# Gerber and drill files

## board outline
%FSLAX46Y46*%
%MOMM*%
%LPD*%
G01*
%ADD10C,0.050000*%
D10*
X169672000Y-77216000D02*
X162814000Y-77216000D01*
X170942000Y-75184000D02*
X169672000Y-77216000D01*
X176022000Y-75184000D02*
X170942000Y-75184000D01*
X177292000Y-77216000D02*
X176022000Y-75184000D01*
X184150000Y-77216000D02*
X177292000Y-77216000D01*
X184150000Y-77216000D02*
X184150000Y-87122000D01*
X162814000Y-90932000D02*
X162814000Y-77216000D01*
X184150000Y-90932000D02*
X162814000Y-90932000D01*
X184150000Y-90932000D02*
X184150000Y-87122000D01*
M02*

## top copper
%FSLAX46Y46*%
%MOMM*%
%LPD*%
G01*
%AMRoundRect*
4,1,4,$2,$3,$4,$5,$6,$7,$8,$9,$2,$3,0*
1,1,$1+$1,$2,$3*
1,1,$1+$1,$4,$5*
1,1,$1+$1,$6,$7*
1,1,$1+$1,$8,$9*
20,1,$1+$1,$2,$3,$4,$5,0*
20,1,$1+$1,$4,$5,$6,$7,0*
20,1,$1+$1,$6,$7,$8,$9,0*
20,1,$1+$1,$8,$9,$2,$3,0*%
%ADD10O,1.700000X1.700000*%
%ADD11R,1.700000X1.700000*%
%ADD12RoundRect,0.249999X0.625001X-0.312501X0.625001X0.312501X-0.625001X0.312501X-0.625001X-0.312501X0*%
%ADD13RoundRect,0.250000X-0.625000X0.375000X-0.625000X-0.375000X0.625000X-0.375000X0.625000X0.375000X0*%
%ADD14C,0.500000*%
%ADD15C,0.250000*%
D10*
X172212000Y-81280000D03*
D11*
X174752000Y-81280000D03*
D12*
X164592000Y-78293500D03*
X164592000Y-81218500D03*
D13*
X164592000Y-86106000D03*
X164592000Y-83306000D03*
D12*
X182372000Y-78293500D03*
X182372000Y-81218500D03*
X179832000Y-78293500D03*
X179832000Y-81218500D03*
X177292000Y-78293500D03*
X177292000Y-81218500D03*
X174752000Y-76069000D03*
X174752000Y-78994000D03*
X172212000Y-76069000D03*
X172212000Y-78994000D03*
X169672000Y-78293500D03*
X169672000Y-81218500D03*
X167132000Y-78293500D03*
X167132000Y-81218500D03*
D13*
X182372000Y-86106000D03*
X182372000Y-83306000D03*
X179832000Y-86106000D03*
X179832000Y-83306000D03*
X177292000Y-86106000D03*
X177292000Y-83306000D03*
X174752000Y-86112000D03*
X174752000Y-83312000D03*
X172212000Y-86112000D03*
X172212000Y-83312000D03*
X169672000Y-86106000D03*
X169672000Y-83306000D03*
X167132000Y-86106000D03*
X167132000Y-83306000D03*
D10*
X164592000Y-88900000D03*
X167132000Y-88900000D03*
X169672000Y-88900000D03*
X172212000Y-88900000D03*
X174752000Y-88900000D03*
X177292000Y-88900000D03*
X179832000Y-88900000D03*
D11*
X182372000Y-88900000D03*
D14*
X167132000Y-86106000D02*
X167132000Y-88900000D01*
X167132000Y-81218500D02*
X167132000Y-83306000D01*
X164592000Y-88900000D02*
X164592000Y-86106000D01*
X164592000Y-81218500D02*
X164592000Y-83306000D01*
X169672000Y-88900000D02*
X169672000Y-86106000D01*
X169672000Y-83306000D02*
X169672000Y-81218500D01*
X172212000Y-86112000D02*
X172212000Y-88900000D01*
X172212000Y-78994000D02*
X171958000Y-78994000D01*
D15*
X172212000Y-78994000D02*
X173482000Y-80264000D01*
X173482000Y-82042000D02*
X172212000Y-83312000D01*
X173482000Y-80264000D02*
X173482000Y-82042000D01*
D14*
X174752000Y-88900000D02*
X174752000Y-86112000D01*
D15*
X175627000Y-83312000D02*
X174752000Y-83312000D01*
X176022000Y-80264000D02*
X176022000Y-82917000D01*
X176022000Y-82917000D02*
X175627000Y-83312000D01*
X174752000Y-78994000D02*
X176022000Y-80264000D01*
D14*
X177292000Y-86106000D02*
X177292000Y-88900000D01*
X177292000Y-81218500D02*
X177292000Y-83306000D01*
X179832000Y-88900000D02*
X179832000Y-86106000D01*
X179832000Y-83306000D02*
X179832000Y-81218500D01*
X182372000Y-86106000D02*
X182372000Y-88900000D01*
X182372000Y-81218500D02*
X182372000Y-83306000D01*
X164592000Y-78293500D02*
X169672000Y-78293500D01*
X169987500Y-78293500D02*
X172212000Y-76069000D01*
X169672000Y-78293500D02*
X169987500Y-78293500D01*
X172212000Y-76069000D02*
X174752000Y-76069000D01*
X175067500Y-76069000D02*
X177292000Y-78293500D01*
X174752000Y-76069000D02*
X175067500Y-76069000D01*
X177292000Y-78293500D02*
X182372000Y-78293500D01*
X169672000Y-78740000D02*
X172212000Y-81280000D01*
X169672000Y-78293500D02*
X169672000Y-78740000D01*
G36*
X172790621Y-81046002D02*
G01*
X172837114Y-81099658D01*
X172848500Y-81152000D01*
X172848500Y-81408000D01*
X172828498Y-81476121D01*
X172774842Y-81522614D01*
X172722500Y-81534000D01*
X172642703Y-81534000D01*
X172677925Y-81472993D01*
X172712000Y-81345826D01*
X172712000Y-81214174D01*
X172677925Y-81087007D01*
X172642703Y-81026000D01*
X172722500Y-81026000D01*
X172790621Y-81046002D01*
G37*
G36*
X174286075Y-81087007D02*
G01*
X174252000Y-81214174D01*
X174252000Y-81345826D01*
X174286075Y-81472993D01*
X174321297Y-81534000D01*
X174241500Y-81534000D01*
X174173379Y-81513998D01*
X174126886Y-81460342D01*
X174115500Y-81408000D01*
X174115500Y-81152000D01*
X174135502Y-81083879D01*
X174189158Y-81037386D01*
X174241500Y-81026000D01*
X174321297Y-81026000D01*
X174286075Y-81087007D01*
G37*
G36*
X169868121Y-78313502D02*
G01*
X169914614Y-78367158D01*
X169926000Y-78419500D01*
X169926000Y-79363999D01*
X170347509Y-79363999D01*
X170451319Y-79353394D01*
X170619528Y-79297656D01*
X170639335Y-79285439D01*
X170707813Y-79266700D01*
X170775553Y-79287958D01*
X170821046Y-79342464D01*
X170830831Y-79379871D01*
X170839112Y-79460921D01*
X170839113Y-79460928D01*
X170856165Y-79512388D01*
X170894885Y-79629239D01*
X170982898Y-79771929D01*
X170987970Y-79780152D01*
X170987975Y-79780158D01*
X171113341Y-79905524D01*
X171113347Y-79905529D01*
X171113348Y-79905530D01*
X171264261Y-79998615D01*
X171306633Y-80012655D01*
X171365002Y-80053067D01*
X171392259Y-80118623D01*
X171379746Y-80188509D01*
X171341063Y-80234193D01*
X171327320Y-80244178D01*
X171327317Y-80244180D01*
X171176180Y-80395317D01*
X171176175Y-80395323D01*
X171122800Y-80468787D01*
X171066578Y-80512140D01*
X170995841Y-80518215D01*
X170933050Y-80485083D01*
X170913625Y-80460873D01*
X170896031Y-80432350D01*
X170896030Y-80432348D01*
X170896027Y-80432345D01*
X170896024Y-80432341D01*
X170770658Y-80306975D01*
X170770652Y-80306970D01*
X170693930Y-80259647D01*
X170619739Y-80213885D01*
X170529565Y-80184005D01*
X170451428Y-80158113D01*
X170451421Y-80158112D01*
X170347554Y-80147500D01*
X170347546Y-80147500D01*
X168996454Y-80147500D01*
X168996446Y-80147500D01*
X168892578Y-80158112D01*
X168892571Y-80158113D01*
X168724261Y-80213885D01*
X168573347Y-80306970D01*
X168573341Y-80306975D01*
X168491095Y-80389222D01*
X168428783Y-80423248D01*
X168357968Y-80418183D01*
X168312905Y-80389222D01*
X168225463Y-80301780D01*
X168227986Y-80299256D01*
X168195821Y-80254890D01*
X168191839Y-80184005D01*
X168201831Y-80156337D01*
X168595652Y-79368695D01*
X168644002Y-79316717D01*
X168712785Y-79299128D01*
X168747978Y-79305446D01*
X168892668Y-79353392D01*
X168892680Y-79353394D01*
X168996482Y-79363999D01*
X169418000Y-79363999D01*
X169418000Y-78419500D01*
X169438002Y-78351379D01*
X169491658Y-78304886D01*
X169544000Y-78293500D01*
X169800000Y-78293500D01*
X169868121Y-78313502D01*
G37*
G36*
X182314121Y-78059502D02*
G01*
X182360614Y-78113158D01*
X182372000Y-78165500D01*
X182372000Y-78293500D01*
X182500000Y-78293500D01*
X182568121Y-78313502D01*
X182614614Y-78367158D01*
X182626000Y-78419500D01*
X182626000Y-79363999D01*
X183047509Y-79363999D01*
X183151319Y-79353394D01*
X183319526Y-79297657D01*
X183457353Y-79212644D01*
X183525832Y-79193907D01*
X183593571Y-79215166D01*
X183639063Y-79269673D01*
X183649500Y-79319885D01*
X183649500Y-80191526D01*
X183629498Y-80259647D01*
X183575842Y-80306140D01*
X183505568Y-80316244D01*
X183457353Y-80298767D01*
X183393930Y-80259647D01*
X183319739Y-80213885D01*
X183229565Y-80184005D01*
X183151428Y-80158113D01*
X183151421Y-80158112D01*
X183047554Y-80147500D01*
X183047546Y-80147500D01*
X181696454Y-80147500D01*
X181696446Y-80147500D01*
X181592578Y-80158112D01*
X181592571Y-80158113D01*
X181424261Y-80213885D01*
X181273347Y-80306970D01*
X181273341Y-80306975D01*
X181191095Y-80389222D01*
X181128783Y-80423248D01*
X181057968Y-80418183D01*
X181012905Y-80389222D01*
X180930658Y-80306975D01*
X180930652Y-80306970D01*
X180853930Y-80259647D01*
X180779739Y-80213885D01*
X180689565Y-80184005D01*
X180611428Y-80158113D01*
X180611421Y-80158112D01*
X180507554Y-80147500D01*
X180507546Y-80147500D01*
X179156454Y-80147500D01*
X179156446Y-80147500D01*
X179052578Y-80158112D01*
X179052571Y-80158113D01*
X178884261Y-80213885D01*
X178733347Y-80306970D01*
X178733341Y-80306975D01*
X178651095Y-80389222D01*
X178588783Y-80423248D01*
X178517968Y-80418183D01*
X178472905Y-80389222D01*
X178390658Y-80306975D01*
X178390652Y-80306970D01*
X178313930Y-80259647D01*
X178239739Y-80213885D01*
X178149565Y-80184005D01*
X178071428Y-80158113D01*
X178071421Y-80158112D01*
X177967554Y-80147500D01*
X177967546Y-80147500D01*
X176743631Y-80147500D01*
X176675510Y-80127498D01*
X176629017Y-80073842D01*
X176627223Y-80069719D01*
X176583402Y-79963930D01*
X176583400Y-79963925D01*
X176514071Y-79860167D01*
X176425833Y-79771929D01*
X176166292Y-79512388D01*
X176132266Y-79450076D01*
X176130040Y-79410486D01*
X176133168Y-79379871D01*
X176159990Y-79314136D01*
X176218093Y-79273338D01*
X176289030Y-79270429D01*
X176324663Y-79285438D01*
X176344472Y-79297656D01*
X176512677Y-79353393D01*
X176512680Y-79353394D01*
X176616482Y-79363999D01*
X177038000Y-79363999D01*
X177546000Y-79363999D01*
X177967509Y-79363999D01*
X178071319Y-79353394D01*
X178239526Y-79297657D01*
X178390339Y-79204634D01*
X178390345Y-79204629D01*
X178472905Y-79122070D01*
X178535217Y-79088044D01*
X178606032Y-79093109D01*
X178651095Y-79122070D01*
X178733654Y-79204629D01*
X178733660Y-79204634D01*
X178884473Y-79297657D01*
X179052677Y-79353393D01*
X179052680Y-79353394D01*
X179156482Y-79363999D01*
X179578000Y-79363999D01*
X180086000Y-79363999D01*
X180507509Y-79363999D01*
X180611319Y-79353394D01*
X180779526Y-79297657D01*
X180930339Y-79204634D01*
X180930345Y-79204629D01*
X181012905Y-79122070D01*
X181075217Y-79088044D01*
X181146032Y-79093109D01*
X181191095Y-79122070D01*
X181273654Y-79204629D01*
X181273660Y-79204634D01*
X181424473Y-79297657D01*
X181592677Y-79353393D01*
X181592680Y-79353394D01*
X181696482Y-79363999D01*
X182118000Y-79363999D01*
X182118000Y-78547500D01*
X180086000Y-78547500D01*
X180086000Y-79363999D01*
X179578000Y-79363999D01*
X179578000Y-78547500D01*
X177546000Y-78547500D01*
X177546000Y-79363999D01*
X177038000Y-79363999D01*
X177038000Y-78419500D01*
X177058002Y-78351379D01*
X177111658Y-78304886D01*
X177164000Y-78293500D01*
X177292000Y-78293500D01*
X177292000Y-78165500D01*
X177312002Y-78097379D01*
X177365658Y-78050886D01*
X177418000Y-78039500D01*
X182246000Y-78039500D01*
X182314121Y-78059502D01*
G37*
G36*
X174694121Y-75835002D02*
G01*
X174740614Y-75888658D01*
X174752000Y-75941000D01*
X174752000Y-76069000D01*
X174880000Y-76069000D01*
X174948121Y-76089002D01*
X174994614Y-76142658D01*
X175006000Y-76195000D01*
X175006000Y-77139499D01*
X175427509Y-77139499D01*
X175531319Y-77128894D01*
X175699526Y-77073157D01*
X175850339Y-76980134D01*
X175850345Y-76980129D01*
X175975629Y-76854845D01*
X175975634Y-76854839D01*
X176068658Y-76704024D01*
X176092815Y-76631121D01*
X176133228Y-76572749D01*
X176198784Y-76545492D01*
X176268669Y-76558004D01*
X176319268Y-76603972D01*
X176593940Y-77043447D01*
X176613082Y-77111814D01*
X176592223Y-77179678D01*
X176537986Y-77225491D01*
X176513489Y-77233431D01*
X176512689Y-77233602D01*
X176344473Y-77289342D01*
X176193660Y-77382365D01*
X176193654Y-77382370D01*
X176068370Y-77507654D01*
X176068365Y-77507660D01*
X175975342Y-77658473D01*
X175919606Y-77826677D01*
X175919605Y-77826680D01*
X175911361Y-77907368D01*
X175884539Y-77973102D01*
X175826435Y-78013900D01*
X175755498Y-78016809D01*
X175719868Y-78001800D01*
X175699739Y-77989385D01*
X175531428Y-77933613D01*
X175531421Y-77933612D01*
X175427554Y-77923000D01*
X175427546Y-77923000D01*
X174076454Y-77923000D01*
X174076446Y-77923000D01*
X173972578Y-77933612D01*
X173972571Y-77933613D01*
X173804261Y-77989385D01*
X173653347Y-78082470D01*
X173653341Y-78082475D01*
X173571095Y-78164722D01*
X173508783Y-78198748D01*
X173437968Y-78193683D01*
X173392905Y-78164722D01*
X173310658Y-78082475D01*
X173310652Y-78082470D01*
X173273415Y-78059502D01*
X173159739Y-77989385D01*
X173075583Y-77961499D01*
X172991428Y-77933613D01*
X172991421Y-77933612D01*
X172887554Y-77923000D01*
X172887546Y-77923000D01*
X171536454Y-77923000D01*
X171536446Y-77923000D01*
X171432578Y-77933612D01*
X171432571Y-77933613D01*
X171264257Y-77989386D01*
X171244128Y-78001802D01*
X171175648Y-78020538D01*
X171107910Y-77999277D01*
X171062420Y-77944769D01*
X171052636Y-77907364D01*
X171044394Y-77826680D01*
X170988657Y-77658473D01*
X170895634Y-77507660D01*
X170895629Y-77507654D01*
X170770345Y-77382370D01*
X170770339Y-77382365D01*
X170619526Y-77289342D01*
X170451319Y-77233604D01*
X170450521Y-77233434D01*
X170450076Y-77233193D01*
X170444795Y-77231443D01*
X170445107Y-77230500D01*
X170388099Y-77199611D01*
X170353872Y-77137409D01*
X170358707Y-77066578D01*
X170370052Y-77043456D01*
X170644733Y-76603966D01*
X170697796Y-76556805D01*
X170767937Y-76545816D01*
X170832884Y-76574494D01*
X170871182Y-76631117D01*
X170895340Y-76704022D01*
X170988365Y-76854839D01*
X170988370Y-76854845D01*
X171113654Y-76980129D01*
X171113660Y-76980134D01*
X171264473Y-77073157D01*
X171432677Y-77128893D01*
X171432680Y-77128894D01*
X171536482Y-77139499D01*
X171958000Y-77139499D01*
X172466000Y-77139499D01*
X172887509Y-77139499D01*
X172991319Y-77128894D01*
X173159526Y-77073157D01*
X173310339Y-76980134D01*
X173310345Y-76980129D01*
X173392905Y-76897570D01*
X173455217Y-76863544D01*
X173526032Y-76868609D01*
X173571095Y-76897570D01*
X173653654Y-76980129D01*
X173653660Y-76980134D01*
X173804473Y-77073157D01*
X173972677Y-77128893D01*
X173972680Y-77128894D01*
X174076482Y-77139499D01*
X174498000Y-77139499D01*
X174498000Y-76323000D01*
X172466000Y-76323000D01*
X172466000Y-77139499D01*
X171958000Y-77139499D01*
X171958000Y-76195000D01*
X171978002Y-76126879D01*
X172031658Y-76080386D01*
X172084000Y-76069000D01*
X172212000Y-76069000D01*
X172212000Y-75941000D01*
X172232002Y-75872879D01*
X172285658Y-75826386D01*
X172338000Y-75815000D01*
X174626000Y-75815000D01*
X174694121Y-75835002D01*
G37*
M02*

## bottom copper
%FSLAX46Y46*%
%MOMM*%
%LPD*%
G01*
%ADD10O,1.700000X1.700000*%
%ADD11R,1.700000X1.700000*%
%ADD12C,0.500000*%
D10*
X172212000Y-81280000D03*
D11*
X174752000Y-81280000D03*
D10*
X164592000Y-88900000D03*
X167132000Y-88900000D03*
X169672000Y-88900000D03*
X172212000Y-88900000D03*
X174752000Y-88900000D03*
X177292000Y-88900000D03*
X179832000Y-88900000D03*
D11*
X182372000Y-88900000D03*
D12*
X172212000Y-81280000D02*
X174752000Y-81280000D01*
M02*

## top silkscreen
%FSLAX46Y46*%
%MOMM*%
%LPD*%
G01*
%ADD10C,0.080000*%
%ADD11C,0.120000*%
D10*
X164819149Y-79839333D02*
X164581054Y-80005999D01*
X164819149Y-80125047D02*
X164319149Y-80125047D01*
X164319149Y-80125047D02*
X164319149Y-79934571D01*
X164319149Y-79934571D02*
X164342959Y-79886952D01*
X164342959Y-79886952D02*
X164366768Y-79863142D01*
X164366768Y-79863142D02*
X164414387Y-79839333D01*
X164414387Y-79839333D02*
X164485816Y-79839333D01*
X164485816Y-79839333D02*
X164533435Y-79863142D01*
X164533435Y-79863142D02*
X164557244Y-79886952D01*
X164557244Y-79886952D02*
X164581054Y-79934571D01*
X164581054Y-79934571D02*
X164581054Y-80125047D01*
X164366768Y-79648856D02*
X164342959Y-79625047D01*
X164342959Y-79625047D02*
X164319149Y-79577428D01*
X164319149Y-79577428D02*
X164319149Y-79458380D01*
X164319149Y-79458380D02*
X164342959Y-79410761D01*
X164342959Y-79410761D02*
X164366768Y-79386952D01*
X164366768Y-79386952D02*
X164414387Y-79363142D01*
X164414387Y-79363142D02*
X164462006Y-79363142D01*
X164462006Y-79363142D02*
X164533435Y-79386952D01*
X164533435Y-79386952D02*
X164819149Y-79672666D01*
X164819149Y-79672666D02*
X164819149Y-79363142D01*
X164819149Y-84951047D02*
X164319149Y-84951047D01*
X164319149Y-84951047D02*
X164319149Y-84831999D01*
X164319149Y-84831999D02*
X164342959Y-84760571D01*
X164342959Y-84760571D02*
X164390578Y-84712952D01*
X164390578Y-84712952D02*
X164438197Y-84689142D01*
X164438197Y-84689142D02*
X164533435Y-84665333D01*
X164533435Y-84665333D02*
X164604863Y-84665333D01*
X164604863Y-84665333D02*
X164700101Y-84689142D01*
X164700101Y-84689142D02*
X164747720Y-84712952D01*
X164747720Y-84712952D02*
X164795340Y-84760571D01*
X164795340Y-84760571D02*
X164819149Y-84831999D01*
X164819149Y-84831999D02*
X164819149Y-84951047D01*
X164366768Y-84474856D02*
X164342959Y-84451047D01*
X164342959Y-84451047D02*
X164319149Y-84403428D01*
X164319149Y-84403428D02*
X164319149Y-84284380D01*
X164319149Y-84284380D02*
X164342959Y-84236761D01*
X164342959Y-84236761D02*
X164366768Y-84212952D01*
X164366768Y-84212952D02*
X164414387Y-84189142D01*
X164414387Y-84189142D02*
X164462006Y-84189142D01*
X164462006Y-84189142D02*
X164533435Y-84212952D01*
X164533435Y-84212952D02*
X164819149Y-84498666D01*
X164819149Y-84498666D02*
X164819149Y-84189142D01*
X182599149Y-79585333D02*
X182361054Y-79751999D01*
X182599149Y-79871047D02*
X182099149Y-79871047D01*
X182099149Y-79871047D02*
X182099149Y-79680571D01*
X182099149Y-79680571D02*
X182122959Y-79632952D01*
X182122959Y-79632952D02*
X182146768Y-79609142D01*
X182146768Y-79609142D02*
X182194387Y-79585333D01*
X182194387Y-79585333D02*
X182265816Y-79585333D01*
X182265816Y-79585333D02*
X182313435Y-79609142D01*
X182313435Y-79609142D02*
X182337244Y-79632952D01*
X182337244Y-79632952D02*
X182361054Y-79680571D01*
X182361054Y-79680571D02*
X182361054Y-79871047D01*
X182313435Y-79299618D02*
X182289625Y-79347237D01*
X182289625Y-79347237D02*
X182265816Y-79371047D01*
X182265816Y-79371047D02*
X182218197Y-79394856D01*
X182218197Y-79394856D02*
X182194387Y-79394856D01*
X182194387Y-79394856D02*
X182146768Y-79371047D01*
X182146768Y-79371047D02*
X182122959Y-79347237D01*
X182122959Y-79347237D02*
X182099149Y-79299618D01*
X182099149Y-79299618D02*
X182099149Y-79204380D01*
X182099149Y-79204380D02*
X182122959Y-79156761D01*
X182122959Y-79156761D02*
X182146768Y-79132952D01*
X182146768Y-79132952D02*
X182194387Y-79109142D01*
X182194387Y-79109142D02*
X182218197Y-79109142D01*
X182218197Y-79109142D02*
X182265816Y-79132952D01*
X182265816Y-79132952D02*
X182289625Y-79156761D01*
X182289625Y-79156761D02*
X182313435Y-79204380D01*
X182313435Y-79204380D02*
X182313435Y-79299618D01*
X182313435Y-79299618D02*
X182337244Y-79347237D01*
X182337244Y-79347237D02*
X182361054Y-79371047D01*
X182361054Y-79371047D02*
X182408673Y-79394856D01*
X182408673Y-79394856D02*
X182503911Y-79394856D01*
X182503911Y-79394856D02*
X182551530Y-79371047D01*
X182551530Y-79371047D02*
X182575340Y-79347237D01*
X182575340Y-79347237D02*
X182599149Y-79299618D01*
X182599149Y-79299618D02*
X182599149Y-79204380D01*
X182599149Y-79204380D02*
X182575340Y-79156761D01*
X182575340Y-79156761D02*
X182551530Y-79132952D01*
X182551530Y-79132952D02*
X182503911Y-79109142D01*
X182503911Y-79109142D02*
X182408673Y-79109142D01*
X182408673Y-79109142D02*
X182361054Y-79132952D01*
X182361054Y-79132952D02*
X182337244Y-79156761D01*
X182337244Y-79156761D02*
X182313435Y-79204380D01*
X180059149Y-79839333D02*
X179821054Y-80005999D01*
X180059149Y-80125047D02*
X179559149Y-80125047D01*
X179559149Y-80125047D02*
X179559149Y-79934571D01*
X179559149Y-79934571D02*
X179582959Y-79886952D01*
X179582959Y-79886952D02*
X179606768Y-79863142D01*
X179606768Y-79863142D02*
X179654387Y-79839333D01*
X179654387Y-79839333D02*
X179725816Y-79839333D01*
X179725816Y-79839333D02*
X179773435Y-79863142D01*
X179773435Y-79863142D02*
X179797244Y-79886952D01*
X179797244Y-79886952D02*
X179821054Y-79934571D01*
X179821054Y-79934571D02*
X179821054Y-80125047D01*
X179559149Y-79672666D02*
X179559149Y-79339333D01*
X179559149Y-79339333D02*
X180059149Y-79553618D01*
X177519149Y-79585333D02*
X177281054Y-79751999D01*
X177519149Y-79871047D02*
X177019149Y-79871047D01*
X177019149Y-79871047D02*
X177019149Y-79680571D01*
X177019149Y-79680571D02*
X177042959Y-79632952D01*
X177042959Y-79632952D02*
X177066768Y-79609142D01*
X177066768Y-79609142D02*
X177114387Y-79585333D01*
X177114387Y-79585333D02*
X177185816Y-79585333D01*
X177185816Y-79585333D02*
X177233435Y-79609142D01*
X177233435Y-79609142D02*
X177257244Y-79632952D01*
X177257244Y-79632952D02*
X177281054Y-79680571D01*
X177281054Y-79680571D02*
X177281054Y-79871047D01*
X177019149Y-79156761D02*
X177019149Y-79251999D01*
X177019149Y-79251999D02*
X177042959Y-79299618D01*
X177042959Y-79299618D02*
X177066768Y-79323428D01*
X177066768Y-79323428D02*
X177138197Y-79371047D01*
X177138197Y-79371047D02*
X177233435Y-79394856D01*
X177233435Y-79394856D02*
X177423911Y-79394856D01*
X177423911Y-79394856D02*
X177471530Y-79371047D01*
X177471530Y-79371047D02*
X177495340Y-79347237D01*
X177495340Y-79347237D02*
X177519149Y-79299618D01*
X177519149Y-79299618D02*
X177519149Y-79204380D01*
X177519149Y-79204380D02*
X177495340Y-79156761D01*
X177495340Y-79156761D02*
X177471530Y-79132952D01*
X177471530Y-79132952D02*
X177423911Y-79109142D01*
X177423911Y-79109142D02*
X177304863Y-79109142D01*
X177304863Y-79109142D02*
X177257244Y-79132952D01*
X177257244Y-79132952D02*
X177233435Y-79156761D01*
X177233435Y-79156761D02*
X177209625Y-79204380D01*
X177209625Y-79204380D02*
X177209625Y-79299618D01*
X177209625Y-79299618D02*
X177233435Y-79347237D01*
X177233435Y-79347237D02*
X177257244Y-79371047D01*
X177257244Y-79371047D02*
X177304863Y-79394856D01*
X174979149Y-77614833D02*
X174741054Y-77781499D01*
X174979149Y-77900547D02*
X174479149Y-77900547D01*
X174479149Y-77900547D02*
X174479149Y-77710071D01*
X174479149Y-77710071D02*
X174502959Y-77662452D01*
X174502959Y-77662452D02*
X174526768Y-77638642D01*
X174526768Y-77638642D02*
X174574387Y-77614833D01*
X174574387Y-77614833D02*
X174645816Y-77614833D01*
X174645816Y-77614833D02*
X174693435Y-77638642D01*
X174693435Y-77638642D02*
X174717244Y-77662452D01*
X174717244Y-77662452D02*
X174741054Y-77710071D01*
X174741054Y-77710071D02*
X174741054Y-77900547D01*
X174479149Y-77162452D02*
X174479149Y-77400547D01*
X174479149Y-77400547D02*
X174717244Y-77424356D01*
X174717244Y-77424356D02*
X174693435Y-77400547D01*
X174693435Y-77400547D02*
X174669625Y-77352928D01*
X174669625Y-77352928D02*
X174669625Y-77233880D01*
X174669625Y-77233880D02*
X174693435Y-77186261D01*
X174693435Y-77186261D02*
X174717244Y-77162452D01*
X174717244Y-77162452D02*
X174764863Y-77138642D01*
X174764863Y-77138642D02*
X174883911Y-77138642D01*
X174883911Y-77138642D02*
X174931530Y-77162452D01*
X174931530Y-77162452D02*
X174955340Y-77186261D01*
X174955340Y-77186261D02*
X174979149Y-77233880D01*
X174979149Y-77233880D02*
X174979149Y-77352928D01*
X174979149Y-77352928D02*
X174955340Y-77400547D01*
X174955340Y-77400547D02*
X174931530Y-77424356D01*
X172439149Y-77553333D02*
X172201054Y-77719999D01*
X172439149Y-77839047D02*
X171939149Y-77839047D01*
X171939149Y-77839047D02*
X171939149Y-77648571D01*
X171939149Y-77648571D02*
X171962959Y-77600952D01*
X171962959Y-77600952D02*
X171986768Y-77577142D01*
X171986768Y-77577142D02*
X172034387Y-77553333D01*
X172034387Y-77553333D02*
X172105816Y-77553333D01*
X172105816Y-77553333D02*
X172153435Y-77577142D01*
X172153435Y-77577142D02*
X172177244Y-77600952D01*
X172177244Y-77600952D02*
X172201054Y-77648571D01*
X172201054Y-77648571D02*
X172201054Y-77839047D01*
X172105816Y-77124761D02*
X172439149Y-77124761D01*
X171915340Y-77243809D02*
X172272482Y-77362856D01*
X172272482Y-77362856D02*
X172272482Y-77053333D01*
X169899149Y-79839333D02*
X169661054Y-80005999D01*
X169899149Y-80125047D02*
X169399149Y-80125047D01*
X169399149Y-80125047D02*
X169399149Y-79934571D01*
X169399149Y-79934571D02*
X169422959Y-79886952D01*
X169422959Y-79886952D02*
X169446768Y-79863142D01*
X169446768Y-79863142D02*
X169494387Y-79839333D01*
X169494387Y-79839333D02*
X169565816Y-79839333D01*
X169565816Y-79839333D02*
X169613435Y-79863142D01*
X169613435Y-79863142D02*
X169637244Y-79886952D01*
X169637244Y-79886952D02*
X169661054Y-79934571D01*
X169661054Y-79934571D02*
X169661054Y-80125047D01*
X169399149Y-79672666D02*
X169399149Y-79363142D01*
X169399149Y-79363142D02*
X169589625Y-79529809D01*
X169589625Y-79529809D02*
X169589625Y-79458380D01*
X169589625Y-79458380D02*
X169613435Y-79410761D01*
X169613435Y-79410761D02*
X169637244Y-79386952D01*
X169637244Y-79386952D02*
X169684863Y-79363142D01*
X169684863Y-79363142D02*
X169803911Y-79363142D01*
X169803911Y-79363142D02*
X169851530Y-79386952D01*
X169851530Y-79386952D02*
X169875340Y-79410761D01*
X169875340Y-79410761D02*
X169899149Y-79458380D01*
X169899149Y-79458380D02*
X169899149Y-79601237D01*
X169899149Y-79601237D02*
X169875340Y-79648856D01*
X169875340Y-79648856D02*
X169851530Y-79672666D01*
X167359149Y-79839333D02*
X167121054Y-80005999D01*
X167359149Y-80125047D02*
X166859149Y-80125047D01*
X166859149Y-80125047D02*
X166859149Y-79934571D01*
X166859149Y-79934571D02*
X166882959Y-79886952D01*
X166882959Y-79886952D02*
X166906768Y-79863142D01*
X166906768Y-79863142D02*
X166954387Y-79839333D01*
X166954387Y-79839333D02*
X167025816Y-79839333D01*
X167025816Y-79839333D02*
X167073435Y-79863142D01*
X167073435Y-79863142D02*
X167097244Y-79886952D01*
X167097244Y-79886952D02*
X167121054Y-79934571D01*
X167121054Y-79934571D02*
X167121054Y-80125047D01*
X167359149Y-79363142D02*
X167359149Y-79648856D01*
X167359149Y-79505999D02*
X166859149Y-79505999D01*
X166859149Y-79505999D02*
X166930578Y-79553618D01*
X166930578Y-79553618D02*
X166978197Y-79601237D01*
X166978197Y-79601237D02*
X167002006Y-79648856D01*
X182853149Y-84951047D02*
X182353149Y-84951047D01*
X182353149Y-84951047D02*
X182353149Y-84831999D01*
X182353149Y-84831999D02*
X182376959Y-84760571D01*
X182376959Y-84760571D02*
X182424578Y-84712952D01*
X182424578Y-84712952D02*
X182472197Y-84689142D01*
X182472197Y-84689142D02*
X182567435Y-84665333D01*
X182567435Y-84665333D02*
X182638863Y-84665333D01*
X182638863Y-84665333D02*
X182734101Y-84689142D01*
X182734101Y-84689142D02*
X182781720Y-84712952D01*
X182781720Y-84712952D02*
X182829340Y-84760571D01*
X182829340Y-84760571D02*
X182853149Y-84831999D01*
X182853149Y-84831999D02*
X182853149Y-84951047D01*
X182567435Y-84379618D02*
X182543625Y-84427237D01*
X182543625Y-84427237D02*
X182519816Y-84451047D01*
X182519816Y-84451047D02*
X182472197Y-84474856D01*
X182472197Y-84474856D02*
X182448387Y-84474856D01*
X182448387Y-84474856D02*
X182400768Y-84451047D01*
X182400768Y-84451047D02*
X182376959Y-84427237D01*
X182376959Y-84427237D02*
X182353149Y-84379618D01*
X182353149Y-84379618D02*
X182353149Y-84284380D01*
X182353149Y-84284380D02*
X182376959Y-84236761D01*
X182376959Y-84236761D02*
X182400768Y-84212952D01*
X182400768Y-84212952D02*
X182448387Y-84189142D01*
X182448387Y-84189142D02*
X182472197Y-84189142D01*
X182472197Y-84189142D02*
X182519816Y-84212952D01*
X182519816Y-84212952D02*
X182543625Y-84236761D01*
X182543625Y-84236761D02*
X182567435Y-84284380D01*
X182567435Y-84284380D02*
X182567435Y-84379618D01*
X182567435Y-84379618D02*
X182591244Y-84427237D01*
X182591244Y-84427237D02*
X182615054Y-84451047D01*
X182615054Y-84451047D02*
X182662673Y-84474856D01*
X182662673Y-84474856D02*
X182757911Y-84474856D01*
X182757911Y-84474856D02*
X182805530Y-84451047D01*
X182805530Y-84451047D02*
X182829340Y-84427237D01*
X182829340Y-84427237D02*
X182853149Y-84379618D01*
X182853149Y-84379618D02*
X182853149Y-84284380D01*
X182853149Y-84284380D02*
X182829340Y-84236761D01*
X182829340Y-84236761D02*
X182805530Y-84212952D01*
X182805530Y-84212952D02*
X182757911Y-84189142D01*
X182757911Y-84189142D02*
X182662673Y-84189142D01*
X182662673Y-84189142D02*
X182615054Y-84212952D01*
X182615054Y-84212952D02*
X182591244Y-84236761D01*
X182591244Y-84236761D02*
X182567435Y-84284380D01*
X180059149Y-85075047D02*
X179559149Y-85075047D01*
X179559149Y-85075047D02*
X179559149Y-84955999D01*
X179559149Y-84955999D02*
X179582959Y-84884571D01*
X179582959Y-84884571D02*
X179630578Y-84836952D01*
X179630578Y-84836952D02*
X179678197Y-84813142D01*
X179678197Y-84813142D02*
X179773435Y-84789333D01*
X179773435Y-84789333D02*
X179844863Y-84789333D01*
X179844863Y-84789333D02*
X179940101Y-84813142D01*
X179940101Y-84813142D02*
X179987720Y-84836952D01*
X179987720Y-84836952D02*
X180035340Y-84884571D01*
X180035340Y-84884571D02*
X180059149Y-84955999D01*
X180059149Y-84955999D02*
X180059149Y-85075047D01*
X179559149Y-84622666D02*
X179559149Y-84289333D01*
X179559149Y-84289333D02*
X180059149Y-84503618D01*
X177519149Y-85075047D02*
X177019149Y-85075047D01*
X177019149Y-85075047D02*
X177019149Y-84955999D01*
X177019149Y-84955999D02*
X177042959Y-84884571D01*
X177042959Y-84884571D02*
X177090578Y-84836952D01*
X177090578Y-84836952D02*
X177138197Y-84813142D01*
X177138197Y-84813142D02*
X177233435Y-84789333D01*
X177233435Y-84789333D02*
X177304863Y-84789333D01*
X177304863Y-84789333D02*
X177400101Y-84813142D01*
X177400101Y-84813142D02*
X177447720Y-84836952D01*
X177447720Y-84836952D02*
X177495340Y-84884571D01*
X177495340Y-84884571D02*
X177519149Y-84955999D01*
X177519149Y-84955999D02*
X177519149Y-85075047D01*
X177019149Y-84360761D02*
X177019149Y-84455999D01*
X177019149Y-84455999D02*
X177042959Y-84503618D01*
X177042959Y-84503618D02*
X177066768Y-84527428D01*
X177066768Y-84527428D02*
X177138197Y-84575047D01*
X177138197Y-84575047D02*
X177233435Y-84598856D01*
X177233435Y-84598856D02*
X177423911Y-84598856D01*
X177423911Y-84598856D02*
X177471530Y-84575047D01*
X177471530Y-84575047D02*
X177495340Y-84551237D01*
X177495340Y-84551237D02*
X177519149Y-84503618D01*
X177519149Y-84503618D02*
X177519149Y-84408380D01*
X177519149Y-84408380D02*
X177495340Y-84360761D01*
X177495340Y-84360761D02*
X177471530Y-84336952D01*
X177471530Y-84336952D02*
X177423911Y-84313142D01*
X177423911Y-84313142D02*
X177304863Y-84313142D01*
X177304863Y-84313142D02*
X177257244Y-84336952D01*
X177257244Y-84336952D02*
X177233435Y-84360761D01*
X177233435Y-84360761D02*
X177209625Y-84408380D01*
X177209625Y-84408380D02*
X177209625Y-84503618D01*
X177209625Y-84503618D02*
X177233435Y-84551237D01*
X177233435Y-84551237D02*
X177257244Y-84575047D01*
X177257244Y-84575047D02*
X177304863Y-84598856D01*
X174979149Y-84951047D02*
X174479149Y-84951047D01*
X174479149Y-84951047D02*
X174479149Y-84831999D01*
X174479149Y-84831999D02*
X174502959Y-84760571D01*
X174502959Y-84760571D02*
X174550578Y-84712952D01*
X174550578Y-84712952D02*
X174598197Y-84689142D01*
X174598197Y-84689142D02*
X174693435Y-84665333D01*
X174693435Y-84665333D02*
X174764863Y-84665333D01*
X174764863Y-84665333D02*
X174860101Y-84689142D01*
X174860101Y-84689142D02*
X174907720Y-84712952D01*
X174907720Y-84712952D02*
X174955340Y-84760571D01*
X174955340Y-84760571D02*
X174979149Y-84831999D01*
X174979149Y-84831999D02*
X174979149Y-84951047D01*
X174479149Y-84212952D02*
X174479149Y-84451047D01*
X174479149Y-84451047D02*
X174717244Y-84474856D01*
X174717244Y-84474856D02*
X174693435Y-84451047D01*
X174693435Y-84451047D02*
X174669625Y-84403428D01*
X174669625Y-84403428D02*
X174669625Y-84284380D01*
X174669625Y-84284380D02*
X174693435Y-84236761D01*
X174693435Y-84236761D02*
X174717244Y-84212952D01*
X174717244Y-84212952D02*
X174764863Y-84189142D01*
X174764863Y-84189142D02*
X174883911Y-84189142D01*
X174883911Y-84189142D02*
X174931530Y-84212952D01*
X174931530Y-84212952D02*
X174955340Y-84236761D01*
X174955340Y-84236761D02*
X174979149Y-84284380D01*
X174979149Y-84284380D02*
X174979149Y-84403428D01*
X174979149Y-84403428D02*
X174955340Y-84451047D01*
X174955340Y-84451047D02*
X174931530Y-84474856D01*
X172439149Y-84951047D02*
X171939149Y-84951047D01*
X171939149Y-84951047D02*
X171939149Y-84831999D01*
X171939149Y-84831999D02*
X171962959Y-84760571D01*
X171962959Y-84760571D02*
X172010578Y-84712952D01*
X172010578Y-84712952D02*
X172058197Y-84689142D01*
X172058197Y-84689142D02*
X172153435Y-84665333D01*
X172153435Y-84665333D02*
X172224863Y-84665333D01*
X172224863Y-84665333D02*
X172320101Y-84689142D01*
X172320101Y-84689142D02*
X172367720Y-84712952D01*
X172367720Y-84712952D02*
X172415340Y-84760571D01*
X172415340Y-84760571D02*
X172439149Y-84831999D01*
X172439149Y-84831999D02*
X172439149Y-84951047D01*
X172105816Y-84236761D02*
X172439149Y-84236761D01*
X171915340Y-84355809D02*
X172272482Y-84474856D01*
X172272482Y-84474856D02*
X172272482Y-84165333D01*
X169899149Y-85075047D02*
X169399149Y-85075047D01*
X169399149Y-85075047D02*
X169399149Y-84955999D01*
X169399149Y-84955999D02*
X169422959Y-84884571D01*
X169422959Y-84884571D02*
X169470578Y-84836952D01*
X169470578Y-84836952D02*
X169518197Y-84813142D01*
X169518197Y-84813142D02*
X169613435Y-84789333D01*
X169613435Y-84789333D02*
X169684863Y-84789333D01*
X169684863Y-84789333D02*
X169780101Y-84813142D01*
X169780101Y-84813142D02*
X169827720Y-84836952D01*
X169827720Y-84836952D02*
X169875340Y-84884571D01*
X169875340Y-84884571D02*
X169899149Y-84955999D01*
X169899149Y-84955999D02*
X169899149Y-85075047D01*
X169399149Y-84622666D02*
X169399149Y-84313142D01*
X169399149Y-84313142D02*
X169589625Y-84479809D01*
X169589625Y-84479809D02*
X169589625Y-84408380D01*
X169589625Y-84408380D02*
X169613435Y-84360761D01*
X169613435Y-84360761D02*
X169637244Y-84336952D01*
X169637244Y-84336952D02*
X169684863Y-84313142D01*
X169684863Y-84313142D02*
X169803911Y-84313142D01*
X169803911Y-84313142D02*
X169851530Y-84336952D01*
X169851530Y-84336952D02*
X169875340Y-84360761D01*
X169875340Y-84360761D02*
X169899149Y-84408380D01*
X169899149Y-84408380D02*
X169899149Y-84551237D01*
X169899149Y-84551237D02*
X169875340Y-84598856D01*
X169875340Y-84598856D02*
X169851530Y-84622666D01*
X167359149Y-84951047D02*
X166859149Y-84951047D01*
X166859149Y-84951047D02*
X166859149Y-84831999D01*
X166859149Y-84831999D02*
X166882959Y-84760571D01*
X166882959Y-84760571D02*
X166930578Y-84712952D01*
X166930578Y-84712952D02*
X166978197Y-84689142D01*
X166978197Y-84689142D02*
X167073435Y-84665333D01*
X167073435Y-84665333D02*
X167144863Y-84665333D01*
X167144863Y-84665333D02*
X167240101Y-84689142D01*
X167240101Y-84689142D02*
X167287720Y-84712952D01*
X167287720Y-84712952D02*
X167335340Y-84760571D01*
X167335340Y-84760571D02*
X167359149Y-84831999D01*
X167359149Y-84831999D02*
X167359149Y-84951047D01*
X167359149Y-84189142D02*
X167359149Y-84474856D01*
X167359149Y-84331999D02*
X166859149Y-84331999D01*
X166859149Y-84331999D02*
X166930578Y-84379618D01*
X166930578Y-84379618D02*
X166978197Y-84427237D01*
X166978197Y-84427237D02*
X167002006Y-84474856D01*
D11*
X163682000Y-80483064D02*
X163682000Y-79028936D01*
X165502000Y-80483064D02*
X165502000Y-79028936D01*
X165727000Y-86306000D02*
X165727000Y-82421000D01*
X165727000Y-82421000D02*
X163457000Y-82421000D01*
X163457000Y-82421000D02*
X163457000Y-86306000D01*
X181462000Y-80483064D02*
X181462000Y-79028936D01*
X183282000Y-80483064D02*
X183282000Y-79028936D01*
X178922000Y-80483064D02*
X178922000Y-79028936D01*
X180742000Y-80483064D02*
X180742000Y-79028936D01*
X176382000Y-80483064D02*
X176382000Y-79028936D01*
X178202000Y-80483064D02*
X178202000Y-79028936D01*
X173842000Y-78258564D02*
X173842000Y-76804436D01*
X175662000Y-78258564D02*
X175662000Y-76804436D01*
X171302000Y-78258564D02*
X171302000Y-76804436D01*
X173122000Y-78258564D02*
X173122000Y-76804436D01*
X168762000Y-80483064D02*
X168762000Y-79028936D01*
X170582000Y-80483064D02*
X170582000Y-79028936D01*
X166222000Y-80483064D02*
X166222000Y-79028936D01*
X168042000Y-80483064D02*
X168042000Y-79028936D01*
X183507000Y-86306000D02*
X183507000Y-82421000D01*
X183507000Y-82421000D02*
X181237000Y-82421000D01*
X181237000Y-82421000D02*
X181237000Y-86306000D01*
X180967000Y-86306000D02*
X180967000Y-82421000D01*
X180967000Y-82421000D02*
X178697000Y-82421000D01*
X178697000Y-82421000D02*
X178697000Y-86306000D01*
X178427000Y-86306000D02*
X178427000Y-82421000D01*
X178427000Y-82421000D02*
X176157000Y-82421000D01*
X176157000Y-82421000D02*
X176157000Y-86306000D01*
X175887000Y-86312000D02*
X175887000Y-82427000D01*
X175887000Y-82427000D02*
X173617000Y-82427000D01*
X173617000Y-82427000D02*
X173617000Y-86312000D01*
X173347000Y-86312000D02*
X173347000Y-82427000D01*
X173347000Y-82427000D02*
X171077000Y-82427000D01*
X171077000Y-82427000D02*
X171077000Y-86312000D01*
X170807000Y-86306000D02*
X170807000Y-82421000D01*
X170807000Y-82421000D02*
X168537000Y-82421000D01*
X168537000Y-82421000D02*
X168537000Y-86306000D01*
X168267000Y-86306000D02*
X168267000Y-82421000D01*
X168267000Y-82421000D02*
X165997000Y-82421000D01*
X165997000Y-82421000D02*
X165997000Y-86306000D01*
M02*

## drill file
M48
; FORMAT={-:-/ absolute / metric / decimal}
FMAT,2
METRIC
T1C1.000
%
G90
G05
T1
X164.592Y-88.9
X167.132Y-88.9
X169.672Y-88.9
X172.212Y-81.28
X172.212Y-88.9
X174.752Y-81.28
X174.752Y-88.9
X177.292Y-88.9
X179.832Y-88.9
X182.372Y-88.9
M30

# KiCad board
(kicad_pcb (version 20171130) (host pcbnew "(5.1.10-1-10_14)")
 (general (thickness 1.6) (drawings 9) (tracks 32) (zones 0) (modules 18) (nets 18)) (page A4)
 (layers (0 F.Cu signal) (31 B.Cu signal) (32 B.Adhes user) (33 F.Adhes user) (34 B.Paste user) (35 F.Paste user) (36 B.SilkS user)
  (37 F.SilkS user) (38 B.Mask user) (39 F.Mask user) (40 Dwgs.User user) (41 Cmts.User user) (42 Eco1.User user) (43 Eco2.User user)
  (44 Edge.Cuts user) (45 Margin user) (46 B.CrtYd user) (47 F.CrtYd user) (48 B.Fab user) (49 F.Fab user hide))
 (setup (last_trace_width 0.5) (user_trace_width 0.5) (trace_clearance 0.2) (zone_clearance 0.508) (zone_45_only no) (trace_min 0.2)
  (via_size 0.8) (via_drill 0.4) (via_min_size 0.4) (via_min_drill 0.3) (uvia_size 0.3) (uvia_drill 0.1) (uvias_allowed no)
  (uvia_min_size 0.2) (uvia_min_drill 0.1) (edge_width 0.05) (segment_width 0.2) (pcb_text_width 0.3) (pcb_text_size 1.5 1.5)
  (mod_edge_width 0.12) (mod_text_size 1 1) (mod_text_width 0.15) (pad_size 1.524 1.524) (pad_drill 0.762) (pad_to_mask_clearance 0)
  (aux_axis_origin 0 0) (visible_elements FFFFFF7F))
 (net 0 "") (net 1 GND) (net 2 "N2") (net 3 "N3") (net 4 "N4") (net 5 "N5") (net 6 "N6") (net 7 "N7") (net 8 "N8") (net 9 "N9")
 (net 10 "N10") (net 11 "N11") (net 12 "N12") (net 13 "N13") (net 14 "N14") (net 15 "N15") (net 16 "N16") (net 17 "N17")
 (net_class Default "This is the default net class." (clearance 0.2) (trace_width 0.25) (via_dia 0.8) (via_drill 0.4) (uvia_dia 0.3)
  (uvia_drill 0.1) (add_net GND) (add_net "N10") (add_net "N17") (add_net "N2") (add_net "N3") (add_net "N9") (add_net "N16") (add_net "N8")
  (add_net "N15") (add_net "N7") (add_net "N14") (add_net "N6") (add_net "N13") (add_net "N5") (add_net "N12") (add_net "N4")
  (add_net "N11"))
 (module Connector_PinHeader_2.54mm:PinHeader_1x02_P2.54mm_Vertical (layer B.Cu) (at 174.752 81.28 90)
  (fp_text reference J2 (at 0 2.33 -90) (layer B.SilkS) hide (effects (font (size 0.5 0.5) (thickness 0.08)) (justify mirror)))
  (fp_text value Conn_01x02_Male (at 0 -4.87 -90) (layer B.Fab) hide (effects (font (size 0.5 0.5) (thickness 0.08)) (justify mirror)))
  (pad 2 thru_hole oval (at 0 -2.54 90) (size 1.7 1.7) (drill 1) (layers *.Cu *.Mask) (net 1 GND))
  (pad 1 thru_hole rect (at 0 0 90) (size 1.7 1.7) (drill 1) (layers *.Cu *.Mask) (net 1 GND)))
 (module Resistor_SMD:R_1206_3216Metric (layer F.Cu) (at 164.592 79.756 90)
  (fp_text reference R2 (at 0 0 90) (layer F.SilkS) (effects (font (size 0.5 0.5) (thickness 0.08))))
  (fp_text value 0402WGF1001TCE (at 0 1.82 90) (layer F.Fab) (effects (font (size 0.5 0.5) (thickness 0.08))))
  (fp_line (start -0.727064 -0.91) (end 0.727064 -0.91) (layer F.SilkS) (width 0.12))
  (fp_line (start -0.727064 0.91) (end 0.727064 0.91) (layer F.SilkS) (width 0.12))
  (pad 2 smd roundrect (at 1.4625 0 90) (size 1.125 1.75) (layers F.Cu F.Paste F.Mask) (roundrect_rratio 0.2222213333333333) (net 1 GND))
  (pad 1 smd roundrect (at -1.4625 0 90) (size 1.125 1.75) (layers F.Cu F.Paste F.Mask) (roundrect_rratio 0.2222213333333333) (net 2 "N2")))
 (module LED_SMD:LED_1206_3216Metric (layer F.Cu) (at 164.592 84.706 270)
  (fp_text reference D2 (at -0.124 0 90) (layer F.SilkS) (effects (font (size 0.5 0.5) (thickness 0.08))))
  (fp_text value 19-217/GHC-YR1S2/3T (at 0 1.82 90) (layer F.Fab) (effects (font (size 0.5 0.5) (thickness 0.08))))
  (fp_line (start 1.6 -1.135) (end -2.285 -1.135) (layer F.SilkS) (width 0.12))
  (fp_line (start -2.285 -1.135) (end -2.285 1.135) (layer F.SilkS) (width 0.12))
  (fp_line (start -2.285 1.135) (end 1.6 1.135) (layer F.SilkS) (width 0.12))
  (pad 2 smd roundrect (at 1.4 0 270) (size 1.25 1.75) (layers F.Cu F.Paste F.Mask) (roundrect_rratio 0.2) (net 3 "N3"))
  (pad 1 smd roundrect (at -1.4 0 270) (size 1.25 1.75) (layers F.Cu F.Paste F.Mask) (roundrect_rratio 0.2) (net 2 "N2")))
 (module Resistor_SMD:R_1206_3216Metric (layer F.Cu) (at 182.372 79.756 90)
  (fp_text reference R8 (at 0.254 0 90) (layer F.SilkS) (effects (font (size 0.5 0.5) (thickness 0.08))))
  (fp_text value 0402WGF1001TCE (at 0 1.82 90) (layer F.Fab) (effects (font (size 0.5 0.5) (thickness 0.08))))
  (fp_line (start -0.727064 -0.91) (end 0.727064 -0.91) (layer F.SilkS) (width 0.12))
  (fp_line (start -0.727064 0.91) (end 0.727064 0.91) (layer F.SilkS) (width 0.12))
  (pad 2 smd roundrect (at 1.4625 0 90) (size 1.125 1.75) (layers F.Cu F.Paste F.Mask) (roundrect_rratio 0.2222213333333333) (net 1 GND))
  (pad 1 smd roundrect (at -1.4625 0 90) (size 1.125 1.75) (layers F.Cu F.Paste F.Mask) (roundrect_rratio 0.2222213333333333) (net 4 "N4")))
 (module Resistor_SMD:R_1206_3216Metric (layer F.Cu) (at 179.832 79.756 90)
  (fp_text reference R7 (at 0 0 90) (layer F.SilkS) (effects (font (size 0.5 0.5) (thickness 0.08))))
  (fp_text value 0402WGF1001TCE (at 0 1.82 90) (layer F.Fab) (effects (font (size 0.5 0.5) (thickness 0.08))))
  (fp_line (start -0.727064 -0.91) (end 0.727064 -0.91) (layer F.SilkS) (width 0.12))
  (fp_line (start -0.727064 0.91) (end 0.727064 0.91) (layer F.SilkS) (width 0.12))
  (pad 2 smd roundrect (at 1.4625 0 90) (size 1.125 1.75) (layers F.Cu F.Paste F.Mask) (roundrect_rratio 0.2222213333333333) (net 1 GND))
  (pad 1 smd roundrect (at -1.4625 0 90) (size 1.125 1.75) (layers F.Cu F.Paste F.Mask) (roundrect_rratio 0.2222213333333333) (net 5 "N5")))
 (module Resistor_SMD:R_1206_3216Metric (layer F.Cu) (at 177.292 79.756 90)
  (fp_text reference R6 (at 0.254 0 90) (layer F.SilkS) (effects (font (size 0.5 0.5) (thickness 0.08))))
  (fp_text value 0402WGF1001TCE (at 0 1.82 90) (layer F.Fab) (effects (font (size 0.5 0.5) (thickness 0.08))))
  (fp_line (start -0.727064 -0.91) (end 0.727064 -0.91) (layer F.SilkS) (width 0.12))
  (fp_line (start -0.727064 0.91) (end 0.727064 0.91) (layer F.SilkS) (width 0.12))
  (pad 2 smd roundrect (at 1.4625 0 90) (size 1.125 1.75) (layers F.Cu F.Paste F.Mask) (roundrect_rratio 0.2222213333333333) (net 1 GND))
  (pad 1 smd roundrect (at -1.4625 0 90) (size 1.125 1.75) (layers F.Cu F.Paste F.Mask) (roundrect_rratio 0.2222213333333333) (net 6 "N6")))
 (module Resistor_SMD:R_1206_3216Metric (layer F.Cu) (at 174.752 77.5315 90)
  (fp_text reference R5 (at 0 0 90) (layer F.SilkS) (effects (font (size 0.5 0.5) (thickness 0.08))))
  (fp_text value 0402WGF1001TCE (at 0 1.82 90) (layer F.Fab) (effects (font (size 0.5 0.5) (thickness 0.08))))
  (fp_line (start -0.727064 -0.91) (end 0.727064 -0.91) (layer F.SilkS) (width 0.12))
  (fp_line (start -0.727064 0.91) (end 0.727064 0.91) (layer F.SilkS) (width 0.12))
  (pad 2 smd roundrect (at 1.4625 0 90) (size 1.125 1.75) (layers F.Cu F.Paste F.Mask) (roundrect_rratio 0.2222213333333333) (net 1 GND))
  (pad 1 smd roundrect (at -1.4625 0 90) (size 1.125 1.75) (layers F.Cu F.Paste F.Mask) (roundrect_rratio 0.2222213333333333) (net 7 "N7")))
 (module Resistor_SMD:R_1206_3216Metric (layer F.Cu) (at 172.212 77.5315 90)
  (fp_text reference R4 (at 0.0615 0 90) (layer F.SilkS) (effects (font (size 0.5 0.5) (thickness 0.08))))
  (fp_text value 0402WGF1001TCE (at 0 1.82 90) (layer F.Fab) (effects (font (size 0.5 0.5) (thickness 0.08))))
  (fp_line (start -0.727064 -0.91) (end 0.727064 -0.91) (layer F.SilkS) (width 0.12))
  (fp_line (start -0.727064 0.91) (end 0.727064 0.91) (layer F.SilkS) (width 0.12))
  (pad 2 smd roundrect (at 1.4625 0 90) (size 1.125 1.75) (layers F.Cu F.Paste F.Mask) (roundrect_rratio 0.2222213333333333) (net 1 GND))
  (pad 1 smd roundrect (at -1.4625 0 90) (size 1.125 1.75) (layers F.Cu F.Paste F.Mask) (roundrect_rratio 0.2222213333333333) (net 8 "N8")))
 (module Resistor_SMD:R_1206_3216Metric (layer F.Cu) (at 169.672 79.756 90)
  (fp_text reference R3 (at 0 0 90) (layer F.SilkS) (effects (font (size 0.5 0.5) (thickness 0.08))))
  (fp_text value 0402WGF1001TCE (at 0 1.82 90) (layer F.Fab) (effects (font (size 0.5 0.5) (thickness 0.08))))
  (fp_line (start -0.727064 -0.91) (end 0.727064 -0.91) (layer F.SilkS) (width 0.12))
  (fp_line (start -0.727064 0.91) (end 0.727064 0.91) (layer F.SilkS) (width 0.12))
  (pad 2 smd roundrect (at 1.4625 0 90) (size 1.125 1.75) (layers F.Cu F.Paste F.Mask) (roundrect_rratio 0.2222213333333333) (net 1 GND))
  (pad 1 smd roundrect (at -1.4625 0 90) (size 1.125 1.75) (layers F.Cu F.Paste F.Mask) (roundrect_rratio 0.2222213333333333) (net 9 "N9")))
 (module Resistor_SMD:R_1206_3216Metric (layer F.Cu) (at 167.132 79.756 90)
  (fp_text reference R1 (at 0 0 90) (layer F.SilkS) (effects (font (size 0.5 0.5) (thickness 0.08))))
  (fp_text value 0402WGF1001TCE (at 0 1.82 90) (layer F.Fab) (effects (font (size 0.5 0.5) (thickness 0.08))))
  (fp_line (start -0.727064 -0.91) (end 0.727064 -0.91) (layer F.SilkS) (width 0.12))
  (fp_line (start -0.727064 0.91) (end 0.727064 0.91) (layer F.SilkS) (width 0.12))
  (pad 2 smd roundrect (at 1.4625 0 90) (size 1.125 1.75) (layers F.Cu F.Paste F.Mask) (roundrect_rratio 0.2222213333333333) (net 1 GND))
  (pad 1 smd roundrect (at -1.4625 0 90) (size 1.125 1.75) (layers F.Cu F.Paste F.Mask) (roundrect_rratio 0.2222213333333333) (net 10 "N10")))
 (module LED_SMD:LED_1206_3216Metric (layer F.Cu) (at 182.372 84.706 270)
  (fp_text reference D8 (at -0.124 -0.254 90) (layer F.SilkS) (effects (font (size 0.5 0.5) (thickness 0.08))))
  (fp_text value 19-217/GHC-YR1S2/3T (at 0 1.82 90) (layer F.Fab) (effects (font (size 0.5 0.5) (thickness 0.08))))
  (fp_line (start 1.6 -1.135) (end -2.285 -1.135) (layer F.SilkS) (width 0.12))
  (fp_line (start -2.285 -1.135) (end -2.285 1.135) (layer F.SilkS) (width 0.12))
  (fp_line (start -2.285 1.135) (end 1.6 1.135) (layer F.SilkS) (width 0.12))
  (pad 2 smd roundrect (at 1.4 0 270) (size 1.25 1.75) (layers F.Cu F.Paste F.Mask) (roundrect_rratio 0.2) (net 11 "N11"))
  (pad 1 smd roundrect (at -1.4 0 270) (size 1.25 1.75) (layers F.Cu F.Paste F.Mask) (roundrect_rratio 0.2) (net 4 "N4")))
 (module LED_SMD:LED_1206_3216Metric (layer F.Cu) (at 179.832 84.706 270)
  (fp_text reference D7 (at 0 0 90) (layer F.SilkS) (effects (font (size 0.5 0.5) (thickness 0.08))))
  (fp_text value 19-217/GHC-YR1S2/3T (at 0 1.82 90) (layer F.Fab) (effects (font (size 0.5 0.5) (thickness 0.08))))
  (fp_line (start 1.6 -1.135) (end -2.285 -1.135) (layer F.SilkS) (width 0.12))
  (fp_line (start -2.285 -1.135) (end -2.285 1.135) (layer F.SilkS) (width 0.12))
  (fp_line (start -2.285 1.135) (end 1.6 1.135) (layer F.SilkS) (width 0.12))
  (pad 2 smd roundrect (at 1.4 0 270) (size 1.25 1.75) (layers F.Cu F.Paste F.Mask) (roundrect_rratio 0.2) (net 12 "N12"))
  (pad 1 smd roundrect (at -1.4 0 270) (size 1.25 1.75) (layers F.Cu F.Paste F.Mask) (roundrect_rratio 0.2) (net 5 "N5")))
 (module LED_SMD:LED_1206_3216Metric (layer F.Cu) (at 177.292 84.706 270)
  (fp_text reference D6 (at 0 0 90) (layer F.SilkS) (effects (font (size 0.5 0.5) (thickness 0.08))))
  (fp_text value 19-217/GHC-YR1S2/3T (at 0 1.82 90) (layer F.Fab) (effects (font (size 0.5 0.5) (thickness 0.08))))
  (fp_line (start 1.6 -1.135) (end -2.285 -1.135) (layer F.SilkS) (width 0.12))
  (fp_line (start -2.285 -1.135) (end -2.285 1.135) (layer F.SilkS) (width 0.12))
  (fp_line (start -2.285 1.135) (end 1.6 1.135) (layer F.SilkS) (width 0.12))
  (pad 2 smd roundrect (at 1.4 0 270) (size 1.25 1.75) (layers F.Cu F.Paste F.Mask) (roundrect_rratio 0.2) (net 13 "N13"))
  (pad 1 smd roundrect (at -1.4 0 270) (size 1.25 1.75) (layers F.Cu F.Paste F.Mask) (roundrect_rratio 0.2) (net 6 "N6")))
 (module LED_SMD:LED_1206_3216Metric (layer F.Cu) (at 174.752 84.712 270)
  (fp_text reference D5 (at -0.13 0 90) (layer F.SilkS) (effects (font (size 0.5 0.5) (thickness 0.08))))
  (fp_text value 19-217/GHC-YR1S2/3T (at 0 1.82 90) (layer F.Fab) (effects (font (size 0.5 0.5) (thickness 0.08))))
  (fp_line (start 1.6 -1.135) (end -2.285 -1.135) (layer F.SilkS) (width 0.12))
  (fp_line (start -2.285 -1.135) (end -2.285 1.135) (layer F.SilkS) (width 0.12))
  (fp_line (start -2.285 1.135) (end 1.6 1.135) (layer F.SilkS) (width 0.12))
  (pad 2 smd roundrect (at 1.4 0 270) (size 1.25 1.75) (layers F.Cu F.Paste F.Mask) (roundrect_rratio 0.2) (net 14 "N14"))
  (pad 1 smd roundrect (at -1.4 0 270) (size 1.25 1.75) (layers F.Cu F.Paste F.Mask) (roundrect_rratio 0.2) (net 7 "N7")))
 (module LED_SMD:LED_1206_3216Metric (layer F.Cu) (at 172.212 84.712 270)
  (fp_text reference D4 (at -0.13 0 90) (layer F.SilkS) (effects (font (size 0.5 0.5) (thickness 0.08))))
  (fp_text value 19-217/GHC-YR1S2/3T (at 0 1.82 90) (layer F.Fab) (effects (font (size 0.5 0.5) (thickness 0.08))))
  (fp_line (start 1.6 -1.135) (end -2.285 -1.135) (layer F.SilkS) (width 0.12))
  (fp_line (start -2.285 -1.135) (end -2.285 1.135) (layer F.SilkS) (width 0.12))
  (fp_line (start -2.285 1.135) (end 1.6 1.135) (layer F.SilkS) (width 0.12))
  (pad 2 smd roundrect (at 1.4 0 270) (size 1.25 1.75) (layers F.Cu F.Paste F.Mask) (roundrect_rratio 0.2) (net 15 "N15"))
  (pad 1 smd roundrect (at -1.4 0 270) (size 1.25 1.75) (layers F.Cu F.Paste F.Mask) (roundrect_rratio 0.2) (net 8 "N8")))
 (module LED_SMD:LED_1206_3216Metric (layer F.Cu) (at 169.672 84.706 270)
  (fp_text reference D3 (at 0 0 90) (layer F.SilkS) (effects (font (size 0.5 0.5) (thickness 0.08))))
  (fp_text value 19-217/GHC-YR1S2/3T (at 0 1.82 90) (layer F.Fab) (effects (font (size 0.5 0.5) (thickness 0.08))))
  (fp_line (start 1.6 -1.135) (end -2.285 -1.135) (layer F.SilkS) (width 0.12))
  (fp_line (start -2.285 -1.135) (end -2.285 1.135) (layer F.SilkS) (width 0.12))
  (fp_line (start -2.285 1.135) (end 1.6 1.135) (layer F.SilkS) (width 0.12))
  (pad 2 smd roundrect (at 1.4 0 270) (size 1.25 1.75) (layers F.Cu F.Paste F.Mask) (roundrect_rratio 0.2) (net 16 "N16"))
  (pad 1 smd roundrect (at -1.4 0 270) (size 1.25 1.75) (layers F.Cu F.Paste F.Mask) (roundrect_rratio 0.2) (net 9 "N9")))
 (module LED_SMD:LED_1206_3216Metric (layer F.Cu) (at 167.132 84.706 270)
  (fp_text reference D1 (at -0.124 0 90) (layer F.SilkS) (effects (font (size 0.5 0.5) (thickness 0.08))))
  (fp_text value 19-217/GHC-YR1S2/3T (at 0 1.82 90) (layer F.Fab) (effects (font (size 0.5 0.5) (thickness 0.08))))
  (fp_line (start 1.6 -1.135) (end -2.285 -1.135) (layer F.SilkS) (width 0.12))
  (fp_line (start -2.285 -1.135) (end -2.285 1.135) (layer F.SilkS) (width 0.12))
  (fp_line (start -2.285 1.135) (end 1.6 1.135) (layer F.SilkS) (width 0.12))
  (pad 2 smd roundrect (at 1.4 0 270) (size 1.25 1.75) (layers F.Cu F.Paste F.Mask) (roundrect_rratio 0.2) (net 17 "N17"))
  (pad 1 smd roundrect (at -1.4 0 270) (size 1.25 1.75) (layers F.Cu F.Paste F.Mask) (roundrect_rratio 0.2) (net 10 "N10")))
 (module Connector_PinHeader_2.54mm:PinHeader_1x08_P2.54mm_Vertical (layer B.Cu) (at 182.372 88.9 90)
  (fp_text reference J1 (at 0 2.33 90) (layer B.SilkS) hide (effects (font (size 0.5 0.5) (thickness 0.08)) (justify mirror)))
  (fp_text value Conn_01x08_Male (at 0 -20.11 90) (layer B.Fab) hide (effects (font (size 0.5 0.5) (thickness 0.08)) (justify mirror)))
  (pad 8 thru_hole oval (at 0 -17.78 90) (size 1.7 1.7) (drill 1) (layers *.Cu *.Mask) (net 3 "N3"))
  (pad 7 thru_hole oval (at 0 -15.24 90) (size 1.7 1.7) (drill 1) (layers *.Cu *.Mask) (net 17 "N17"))
  (pad 6 thru_hole oval (at 0 -12.7 90) (size 1.7 1.7) (drill 1) (layers *.Cu *.Mask) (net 16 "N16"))
  (pad 5 thru_hole oval (at 0 -10.16 90) (size 1.7 1.7) (drill 1) (layers *.Cu *.Mask) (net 15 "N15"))
  (pad 4 thru_hole oval (at 0 -7.62 90) (size 1.7 1.7) (drill 1) (layers *.Cu *.Mask) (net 14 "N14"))
  (pad 3 thru_hole oval (at 0 -5.08 90) (size 1.7 1.7) (drill 1) (layers *.Cu *.Mask) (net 13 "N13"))
  (pad 2 thru_hole oval (at 0 -2.54 90) (size 1.7 1.7) (drill 1) (layers *.Cu *.Mask) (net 12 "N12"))
  (pad 1 thru_hole rect (at 0 0 90) (size 1.7 1.7) (drill 1) (layers *.Cu *.Mask) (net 11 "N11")))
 (gr_line (start 169.672 77.216) (end 162.814 77.216) (layer Edge.Cuts) (width 0.05))
 (gr_line (start 170.942 75.184) (end 169.672 77.216) (layer Edge.Cuts) (width 0.05))
 (gr_line (start 176.022 75.184) (end 170.942 75.184) (layer Edge.Cuts) (width 0.05))
 (gr_line (start 177.292 77.216) (end 176.022 75.184) (layer Edge.Cuts) (width 0.05))
 (gr_line (start 184.15 77.216) (end 177.292 77.216) (layer Edge.Cuts) (width 0.05))
 (gr_line (start 184.15 77.216) (end 184.15 87.122) (layer Edge.Cuts) (width 0.05))
 (gr_line (start 162.814 90.932) (end 162.814 77.216) (layer Edge.Cuts) (width 0.05))
 (gr_line (start 184.15 90.932) (end 162.814 90.932) (layer Edge.Cuts) (width 0.05))
 (gr_line (start 184.15 90.932) (end 184.15 87.122) (layer Edge.Cuts) (width 0.05))
 (segment (start 167.132 86.106) (end 167.132 88.9) (width 0.5) (layer F.Cu) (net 17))
 (segment (start 167.132 81.2185) (end 167.132 83.306) (width 0.5) (layer F.Cu) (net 10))
 (segment (start 164.592 88.9) (end 164.592 86.106) (width 0.5) (layer F.Cu) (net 3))
 (segment (start 164.592 81.2185) (end 164.592 83.306) (width 0.5) (layer F.Cu) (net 2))
 (segment (start 169.672 88.9) (end 169.672 86.106) (width 0.5) (layer F.Cu) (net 16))
 (segment (start 169.672 83.306) (end 169.672 81.2185) (width 0.5) (layer F.Cu) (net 9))
 (segment (start 172.212 86.112) (end 172.212 88.9) (width 0.5) (layer F.Cu) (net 15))
 (segment (start 172.212 78.994) (end 171.958 78.994) (width 0.5) (layer F.Cu) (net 8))
 (segment (start 172.212 78.994) (end 173.482 80.264) (width 0.25) (layer F.Cu) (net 8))
 (segment (start 173.482 82.042) (end 172.212 83.312) (width 0.25) (layer F.Cu) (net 8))
 (segment (start 173.482 80.264) (end 173.482 82.042) (width 0.25) (layer F.Cu) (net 8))
 (segment (start 174.752 88.9) (end 174.752 86.112) (width 0.5) (layer F.Cu) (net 14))
 (segment (start 175.627 83.312) (end 174.752 83.312) (width 0.25) (layer F.Cu) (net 7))
 (segment (start 176.022 80.264) (end 176.022 82.917) (width 0.25) (layer F.Cu) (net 7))
 (segment (start 176.022 82.917) (end 175.627 83.312) (width 0.25) (layer F.Cu) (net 7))
 (segment (start 174.752 78.994) (end 176.022 80.264) (width 0.25) (layer F.Cu) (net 7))
 (segment (start 177.292 86.106) (end 177.292 88.9) (width 0.5) (layer F.Cu) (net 13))
 (segment (start 177.292 81.2185) (end 177.292 83.306) (width 0.5) (layer F.Cu) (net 6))
 (segment (start 179.832 88.9) (end 179.832 86.106) (width 0.5) (layer F.Cu) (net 12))
 (segment (start 179.832 83.306) (end 179.832 81.2185) (width 0.5) (layer F.Cu) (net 5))
 (segment (start 182.372 86.106) (end 182.372 88.9) (width 0.5) (layer F.Cu) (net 11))
 (segment (start 182.372 81.2185) (end 182.372 83.306) (width 0.5) (layer F.Cu) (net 4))
 (segment (start 164.592 78.2935) (end 169.672 78.2935) (width 0.5) (layer F.Cu) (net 1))
 (segment (start 169.9875 78.2935) (end 172.212 76.069) (width 0.5) (layer F.Cu) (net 1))
 (segment (start 169.672 78.2935) (end 169.9875 78.2935) (width 0.5) (layer F.Cu) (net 1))
 (segment (start 172.212 76.069) (end 174.752 76.069) (width 0.5) (layer F.Cu) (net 1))
 (segment (start 175.0675 76.069) (end 177.292 78.2935) (width 0.5) (layer F.Cu) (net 1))
 (segment (start 174.752 76.069) (end 175.0675 76.069) (width 0.5) (layer F.Cu) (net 1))
 (segment (start 177.292 78.2935) (end 182.372 78.2935) (width 0.5) (layer F.Cu) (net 1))
 (segment (start 169.672 78.74) (end 172.212 81.28) (width 0.5) (layer F.Cu) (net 1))
 (segment (start 169.672 78.2935) (end 169.672 78.74) (width 0.5) (layer F.Cu) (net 1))
 (segment (start 172.212 81.28) (end 174.752 81.28) (width 0.5) (layer B.Cu) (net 1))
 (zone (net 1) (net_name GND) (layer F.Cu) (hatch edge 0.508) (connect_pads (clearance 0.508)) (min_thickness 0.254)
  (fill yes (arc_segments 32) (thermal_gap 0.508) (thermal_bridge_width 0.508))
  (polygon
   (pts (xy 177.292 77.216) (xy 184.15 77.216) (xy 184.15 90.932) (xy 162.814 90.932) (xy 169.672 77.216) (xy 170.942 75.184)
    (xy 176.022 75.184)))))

